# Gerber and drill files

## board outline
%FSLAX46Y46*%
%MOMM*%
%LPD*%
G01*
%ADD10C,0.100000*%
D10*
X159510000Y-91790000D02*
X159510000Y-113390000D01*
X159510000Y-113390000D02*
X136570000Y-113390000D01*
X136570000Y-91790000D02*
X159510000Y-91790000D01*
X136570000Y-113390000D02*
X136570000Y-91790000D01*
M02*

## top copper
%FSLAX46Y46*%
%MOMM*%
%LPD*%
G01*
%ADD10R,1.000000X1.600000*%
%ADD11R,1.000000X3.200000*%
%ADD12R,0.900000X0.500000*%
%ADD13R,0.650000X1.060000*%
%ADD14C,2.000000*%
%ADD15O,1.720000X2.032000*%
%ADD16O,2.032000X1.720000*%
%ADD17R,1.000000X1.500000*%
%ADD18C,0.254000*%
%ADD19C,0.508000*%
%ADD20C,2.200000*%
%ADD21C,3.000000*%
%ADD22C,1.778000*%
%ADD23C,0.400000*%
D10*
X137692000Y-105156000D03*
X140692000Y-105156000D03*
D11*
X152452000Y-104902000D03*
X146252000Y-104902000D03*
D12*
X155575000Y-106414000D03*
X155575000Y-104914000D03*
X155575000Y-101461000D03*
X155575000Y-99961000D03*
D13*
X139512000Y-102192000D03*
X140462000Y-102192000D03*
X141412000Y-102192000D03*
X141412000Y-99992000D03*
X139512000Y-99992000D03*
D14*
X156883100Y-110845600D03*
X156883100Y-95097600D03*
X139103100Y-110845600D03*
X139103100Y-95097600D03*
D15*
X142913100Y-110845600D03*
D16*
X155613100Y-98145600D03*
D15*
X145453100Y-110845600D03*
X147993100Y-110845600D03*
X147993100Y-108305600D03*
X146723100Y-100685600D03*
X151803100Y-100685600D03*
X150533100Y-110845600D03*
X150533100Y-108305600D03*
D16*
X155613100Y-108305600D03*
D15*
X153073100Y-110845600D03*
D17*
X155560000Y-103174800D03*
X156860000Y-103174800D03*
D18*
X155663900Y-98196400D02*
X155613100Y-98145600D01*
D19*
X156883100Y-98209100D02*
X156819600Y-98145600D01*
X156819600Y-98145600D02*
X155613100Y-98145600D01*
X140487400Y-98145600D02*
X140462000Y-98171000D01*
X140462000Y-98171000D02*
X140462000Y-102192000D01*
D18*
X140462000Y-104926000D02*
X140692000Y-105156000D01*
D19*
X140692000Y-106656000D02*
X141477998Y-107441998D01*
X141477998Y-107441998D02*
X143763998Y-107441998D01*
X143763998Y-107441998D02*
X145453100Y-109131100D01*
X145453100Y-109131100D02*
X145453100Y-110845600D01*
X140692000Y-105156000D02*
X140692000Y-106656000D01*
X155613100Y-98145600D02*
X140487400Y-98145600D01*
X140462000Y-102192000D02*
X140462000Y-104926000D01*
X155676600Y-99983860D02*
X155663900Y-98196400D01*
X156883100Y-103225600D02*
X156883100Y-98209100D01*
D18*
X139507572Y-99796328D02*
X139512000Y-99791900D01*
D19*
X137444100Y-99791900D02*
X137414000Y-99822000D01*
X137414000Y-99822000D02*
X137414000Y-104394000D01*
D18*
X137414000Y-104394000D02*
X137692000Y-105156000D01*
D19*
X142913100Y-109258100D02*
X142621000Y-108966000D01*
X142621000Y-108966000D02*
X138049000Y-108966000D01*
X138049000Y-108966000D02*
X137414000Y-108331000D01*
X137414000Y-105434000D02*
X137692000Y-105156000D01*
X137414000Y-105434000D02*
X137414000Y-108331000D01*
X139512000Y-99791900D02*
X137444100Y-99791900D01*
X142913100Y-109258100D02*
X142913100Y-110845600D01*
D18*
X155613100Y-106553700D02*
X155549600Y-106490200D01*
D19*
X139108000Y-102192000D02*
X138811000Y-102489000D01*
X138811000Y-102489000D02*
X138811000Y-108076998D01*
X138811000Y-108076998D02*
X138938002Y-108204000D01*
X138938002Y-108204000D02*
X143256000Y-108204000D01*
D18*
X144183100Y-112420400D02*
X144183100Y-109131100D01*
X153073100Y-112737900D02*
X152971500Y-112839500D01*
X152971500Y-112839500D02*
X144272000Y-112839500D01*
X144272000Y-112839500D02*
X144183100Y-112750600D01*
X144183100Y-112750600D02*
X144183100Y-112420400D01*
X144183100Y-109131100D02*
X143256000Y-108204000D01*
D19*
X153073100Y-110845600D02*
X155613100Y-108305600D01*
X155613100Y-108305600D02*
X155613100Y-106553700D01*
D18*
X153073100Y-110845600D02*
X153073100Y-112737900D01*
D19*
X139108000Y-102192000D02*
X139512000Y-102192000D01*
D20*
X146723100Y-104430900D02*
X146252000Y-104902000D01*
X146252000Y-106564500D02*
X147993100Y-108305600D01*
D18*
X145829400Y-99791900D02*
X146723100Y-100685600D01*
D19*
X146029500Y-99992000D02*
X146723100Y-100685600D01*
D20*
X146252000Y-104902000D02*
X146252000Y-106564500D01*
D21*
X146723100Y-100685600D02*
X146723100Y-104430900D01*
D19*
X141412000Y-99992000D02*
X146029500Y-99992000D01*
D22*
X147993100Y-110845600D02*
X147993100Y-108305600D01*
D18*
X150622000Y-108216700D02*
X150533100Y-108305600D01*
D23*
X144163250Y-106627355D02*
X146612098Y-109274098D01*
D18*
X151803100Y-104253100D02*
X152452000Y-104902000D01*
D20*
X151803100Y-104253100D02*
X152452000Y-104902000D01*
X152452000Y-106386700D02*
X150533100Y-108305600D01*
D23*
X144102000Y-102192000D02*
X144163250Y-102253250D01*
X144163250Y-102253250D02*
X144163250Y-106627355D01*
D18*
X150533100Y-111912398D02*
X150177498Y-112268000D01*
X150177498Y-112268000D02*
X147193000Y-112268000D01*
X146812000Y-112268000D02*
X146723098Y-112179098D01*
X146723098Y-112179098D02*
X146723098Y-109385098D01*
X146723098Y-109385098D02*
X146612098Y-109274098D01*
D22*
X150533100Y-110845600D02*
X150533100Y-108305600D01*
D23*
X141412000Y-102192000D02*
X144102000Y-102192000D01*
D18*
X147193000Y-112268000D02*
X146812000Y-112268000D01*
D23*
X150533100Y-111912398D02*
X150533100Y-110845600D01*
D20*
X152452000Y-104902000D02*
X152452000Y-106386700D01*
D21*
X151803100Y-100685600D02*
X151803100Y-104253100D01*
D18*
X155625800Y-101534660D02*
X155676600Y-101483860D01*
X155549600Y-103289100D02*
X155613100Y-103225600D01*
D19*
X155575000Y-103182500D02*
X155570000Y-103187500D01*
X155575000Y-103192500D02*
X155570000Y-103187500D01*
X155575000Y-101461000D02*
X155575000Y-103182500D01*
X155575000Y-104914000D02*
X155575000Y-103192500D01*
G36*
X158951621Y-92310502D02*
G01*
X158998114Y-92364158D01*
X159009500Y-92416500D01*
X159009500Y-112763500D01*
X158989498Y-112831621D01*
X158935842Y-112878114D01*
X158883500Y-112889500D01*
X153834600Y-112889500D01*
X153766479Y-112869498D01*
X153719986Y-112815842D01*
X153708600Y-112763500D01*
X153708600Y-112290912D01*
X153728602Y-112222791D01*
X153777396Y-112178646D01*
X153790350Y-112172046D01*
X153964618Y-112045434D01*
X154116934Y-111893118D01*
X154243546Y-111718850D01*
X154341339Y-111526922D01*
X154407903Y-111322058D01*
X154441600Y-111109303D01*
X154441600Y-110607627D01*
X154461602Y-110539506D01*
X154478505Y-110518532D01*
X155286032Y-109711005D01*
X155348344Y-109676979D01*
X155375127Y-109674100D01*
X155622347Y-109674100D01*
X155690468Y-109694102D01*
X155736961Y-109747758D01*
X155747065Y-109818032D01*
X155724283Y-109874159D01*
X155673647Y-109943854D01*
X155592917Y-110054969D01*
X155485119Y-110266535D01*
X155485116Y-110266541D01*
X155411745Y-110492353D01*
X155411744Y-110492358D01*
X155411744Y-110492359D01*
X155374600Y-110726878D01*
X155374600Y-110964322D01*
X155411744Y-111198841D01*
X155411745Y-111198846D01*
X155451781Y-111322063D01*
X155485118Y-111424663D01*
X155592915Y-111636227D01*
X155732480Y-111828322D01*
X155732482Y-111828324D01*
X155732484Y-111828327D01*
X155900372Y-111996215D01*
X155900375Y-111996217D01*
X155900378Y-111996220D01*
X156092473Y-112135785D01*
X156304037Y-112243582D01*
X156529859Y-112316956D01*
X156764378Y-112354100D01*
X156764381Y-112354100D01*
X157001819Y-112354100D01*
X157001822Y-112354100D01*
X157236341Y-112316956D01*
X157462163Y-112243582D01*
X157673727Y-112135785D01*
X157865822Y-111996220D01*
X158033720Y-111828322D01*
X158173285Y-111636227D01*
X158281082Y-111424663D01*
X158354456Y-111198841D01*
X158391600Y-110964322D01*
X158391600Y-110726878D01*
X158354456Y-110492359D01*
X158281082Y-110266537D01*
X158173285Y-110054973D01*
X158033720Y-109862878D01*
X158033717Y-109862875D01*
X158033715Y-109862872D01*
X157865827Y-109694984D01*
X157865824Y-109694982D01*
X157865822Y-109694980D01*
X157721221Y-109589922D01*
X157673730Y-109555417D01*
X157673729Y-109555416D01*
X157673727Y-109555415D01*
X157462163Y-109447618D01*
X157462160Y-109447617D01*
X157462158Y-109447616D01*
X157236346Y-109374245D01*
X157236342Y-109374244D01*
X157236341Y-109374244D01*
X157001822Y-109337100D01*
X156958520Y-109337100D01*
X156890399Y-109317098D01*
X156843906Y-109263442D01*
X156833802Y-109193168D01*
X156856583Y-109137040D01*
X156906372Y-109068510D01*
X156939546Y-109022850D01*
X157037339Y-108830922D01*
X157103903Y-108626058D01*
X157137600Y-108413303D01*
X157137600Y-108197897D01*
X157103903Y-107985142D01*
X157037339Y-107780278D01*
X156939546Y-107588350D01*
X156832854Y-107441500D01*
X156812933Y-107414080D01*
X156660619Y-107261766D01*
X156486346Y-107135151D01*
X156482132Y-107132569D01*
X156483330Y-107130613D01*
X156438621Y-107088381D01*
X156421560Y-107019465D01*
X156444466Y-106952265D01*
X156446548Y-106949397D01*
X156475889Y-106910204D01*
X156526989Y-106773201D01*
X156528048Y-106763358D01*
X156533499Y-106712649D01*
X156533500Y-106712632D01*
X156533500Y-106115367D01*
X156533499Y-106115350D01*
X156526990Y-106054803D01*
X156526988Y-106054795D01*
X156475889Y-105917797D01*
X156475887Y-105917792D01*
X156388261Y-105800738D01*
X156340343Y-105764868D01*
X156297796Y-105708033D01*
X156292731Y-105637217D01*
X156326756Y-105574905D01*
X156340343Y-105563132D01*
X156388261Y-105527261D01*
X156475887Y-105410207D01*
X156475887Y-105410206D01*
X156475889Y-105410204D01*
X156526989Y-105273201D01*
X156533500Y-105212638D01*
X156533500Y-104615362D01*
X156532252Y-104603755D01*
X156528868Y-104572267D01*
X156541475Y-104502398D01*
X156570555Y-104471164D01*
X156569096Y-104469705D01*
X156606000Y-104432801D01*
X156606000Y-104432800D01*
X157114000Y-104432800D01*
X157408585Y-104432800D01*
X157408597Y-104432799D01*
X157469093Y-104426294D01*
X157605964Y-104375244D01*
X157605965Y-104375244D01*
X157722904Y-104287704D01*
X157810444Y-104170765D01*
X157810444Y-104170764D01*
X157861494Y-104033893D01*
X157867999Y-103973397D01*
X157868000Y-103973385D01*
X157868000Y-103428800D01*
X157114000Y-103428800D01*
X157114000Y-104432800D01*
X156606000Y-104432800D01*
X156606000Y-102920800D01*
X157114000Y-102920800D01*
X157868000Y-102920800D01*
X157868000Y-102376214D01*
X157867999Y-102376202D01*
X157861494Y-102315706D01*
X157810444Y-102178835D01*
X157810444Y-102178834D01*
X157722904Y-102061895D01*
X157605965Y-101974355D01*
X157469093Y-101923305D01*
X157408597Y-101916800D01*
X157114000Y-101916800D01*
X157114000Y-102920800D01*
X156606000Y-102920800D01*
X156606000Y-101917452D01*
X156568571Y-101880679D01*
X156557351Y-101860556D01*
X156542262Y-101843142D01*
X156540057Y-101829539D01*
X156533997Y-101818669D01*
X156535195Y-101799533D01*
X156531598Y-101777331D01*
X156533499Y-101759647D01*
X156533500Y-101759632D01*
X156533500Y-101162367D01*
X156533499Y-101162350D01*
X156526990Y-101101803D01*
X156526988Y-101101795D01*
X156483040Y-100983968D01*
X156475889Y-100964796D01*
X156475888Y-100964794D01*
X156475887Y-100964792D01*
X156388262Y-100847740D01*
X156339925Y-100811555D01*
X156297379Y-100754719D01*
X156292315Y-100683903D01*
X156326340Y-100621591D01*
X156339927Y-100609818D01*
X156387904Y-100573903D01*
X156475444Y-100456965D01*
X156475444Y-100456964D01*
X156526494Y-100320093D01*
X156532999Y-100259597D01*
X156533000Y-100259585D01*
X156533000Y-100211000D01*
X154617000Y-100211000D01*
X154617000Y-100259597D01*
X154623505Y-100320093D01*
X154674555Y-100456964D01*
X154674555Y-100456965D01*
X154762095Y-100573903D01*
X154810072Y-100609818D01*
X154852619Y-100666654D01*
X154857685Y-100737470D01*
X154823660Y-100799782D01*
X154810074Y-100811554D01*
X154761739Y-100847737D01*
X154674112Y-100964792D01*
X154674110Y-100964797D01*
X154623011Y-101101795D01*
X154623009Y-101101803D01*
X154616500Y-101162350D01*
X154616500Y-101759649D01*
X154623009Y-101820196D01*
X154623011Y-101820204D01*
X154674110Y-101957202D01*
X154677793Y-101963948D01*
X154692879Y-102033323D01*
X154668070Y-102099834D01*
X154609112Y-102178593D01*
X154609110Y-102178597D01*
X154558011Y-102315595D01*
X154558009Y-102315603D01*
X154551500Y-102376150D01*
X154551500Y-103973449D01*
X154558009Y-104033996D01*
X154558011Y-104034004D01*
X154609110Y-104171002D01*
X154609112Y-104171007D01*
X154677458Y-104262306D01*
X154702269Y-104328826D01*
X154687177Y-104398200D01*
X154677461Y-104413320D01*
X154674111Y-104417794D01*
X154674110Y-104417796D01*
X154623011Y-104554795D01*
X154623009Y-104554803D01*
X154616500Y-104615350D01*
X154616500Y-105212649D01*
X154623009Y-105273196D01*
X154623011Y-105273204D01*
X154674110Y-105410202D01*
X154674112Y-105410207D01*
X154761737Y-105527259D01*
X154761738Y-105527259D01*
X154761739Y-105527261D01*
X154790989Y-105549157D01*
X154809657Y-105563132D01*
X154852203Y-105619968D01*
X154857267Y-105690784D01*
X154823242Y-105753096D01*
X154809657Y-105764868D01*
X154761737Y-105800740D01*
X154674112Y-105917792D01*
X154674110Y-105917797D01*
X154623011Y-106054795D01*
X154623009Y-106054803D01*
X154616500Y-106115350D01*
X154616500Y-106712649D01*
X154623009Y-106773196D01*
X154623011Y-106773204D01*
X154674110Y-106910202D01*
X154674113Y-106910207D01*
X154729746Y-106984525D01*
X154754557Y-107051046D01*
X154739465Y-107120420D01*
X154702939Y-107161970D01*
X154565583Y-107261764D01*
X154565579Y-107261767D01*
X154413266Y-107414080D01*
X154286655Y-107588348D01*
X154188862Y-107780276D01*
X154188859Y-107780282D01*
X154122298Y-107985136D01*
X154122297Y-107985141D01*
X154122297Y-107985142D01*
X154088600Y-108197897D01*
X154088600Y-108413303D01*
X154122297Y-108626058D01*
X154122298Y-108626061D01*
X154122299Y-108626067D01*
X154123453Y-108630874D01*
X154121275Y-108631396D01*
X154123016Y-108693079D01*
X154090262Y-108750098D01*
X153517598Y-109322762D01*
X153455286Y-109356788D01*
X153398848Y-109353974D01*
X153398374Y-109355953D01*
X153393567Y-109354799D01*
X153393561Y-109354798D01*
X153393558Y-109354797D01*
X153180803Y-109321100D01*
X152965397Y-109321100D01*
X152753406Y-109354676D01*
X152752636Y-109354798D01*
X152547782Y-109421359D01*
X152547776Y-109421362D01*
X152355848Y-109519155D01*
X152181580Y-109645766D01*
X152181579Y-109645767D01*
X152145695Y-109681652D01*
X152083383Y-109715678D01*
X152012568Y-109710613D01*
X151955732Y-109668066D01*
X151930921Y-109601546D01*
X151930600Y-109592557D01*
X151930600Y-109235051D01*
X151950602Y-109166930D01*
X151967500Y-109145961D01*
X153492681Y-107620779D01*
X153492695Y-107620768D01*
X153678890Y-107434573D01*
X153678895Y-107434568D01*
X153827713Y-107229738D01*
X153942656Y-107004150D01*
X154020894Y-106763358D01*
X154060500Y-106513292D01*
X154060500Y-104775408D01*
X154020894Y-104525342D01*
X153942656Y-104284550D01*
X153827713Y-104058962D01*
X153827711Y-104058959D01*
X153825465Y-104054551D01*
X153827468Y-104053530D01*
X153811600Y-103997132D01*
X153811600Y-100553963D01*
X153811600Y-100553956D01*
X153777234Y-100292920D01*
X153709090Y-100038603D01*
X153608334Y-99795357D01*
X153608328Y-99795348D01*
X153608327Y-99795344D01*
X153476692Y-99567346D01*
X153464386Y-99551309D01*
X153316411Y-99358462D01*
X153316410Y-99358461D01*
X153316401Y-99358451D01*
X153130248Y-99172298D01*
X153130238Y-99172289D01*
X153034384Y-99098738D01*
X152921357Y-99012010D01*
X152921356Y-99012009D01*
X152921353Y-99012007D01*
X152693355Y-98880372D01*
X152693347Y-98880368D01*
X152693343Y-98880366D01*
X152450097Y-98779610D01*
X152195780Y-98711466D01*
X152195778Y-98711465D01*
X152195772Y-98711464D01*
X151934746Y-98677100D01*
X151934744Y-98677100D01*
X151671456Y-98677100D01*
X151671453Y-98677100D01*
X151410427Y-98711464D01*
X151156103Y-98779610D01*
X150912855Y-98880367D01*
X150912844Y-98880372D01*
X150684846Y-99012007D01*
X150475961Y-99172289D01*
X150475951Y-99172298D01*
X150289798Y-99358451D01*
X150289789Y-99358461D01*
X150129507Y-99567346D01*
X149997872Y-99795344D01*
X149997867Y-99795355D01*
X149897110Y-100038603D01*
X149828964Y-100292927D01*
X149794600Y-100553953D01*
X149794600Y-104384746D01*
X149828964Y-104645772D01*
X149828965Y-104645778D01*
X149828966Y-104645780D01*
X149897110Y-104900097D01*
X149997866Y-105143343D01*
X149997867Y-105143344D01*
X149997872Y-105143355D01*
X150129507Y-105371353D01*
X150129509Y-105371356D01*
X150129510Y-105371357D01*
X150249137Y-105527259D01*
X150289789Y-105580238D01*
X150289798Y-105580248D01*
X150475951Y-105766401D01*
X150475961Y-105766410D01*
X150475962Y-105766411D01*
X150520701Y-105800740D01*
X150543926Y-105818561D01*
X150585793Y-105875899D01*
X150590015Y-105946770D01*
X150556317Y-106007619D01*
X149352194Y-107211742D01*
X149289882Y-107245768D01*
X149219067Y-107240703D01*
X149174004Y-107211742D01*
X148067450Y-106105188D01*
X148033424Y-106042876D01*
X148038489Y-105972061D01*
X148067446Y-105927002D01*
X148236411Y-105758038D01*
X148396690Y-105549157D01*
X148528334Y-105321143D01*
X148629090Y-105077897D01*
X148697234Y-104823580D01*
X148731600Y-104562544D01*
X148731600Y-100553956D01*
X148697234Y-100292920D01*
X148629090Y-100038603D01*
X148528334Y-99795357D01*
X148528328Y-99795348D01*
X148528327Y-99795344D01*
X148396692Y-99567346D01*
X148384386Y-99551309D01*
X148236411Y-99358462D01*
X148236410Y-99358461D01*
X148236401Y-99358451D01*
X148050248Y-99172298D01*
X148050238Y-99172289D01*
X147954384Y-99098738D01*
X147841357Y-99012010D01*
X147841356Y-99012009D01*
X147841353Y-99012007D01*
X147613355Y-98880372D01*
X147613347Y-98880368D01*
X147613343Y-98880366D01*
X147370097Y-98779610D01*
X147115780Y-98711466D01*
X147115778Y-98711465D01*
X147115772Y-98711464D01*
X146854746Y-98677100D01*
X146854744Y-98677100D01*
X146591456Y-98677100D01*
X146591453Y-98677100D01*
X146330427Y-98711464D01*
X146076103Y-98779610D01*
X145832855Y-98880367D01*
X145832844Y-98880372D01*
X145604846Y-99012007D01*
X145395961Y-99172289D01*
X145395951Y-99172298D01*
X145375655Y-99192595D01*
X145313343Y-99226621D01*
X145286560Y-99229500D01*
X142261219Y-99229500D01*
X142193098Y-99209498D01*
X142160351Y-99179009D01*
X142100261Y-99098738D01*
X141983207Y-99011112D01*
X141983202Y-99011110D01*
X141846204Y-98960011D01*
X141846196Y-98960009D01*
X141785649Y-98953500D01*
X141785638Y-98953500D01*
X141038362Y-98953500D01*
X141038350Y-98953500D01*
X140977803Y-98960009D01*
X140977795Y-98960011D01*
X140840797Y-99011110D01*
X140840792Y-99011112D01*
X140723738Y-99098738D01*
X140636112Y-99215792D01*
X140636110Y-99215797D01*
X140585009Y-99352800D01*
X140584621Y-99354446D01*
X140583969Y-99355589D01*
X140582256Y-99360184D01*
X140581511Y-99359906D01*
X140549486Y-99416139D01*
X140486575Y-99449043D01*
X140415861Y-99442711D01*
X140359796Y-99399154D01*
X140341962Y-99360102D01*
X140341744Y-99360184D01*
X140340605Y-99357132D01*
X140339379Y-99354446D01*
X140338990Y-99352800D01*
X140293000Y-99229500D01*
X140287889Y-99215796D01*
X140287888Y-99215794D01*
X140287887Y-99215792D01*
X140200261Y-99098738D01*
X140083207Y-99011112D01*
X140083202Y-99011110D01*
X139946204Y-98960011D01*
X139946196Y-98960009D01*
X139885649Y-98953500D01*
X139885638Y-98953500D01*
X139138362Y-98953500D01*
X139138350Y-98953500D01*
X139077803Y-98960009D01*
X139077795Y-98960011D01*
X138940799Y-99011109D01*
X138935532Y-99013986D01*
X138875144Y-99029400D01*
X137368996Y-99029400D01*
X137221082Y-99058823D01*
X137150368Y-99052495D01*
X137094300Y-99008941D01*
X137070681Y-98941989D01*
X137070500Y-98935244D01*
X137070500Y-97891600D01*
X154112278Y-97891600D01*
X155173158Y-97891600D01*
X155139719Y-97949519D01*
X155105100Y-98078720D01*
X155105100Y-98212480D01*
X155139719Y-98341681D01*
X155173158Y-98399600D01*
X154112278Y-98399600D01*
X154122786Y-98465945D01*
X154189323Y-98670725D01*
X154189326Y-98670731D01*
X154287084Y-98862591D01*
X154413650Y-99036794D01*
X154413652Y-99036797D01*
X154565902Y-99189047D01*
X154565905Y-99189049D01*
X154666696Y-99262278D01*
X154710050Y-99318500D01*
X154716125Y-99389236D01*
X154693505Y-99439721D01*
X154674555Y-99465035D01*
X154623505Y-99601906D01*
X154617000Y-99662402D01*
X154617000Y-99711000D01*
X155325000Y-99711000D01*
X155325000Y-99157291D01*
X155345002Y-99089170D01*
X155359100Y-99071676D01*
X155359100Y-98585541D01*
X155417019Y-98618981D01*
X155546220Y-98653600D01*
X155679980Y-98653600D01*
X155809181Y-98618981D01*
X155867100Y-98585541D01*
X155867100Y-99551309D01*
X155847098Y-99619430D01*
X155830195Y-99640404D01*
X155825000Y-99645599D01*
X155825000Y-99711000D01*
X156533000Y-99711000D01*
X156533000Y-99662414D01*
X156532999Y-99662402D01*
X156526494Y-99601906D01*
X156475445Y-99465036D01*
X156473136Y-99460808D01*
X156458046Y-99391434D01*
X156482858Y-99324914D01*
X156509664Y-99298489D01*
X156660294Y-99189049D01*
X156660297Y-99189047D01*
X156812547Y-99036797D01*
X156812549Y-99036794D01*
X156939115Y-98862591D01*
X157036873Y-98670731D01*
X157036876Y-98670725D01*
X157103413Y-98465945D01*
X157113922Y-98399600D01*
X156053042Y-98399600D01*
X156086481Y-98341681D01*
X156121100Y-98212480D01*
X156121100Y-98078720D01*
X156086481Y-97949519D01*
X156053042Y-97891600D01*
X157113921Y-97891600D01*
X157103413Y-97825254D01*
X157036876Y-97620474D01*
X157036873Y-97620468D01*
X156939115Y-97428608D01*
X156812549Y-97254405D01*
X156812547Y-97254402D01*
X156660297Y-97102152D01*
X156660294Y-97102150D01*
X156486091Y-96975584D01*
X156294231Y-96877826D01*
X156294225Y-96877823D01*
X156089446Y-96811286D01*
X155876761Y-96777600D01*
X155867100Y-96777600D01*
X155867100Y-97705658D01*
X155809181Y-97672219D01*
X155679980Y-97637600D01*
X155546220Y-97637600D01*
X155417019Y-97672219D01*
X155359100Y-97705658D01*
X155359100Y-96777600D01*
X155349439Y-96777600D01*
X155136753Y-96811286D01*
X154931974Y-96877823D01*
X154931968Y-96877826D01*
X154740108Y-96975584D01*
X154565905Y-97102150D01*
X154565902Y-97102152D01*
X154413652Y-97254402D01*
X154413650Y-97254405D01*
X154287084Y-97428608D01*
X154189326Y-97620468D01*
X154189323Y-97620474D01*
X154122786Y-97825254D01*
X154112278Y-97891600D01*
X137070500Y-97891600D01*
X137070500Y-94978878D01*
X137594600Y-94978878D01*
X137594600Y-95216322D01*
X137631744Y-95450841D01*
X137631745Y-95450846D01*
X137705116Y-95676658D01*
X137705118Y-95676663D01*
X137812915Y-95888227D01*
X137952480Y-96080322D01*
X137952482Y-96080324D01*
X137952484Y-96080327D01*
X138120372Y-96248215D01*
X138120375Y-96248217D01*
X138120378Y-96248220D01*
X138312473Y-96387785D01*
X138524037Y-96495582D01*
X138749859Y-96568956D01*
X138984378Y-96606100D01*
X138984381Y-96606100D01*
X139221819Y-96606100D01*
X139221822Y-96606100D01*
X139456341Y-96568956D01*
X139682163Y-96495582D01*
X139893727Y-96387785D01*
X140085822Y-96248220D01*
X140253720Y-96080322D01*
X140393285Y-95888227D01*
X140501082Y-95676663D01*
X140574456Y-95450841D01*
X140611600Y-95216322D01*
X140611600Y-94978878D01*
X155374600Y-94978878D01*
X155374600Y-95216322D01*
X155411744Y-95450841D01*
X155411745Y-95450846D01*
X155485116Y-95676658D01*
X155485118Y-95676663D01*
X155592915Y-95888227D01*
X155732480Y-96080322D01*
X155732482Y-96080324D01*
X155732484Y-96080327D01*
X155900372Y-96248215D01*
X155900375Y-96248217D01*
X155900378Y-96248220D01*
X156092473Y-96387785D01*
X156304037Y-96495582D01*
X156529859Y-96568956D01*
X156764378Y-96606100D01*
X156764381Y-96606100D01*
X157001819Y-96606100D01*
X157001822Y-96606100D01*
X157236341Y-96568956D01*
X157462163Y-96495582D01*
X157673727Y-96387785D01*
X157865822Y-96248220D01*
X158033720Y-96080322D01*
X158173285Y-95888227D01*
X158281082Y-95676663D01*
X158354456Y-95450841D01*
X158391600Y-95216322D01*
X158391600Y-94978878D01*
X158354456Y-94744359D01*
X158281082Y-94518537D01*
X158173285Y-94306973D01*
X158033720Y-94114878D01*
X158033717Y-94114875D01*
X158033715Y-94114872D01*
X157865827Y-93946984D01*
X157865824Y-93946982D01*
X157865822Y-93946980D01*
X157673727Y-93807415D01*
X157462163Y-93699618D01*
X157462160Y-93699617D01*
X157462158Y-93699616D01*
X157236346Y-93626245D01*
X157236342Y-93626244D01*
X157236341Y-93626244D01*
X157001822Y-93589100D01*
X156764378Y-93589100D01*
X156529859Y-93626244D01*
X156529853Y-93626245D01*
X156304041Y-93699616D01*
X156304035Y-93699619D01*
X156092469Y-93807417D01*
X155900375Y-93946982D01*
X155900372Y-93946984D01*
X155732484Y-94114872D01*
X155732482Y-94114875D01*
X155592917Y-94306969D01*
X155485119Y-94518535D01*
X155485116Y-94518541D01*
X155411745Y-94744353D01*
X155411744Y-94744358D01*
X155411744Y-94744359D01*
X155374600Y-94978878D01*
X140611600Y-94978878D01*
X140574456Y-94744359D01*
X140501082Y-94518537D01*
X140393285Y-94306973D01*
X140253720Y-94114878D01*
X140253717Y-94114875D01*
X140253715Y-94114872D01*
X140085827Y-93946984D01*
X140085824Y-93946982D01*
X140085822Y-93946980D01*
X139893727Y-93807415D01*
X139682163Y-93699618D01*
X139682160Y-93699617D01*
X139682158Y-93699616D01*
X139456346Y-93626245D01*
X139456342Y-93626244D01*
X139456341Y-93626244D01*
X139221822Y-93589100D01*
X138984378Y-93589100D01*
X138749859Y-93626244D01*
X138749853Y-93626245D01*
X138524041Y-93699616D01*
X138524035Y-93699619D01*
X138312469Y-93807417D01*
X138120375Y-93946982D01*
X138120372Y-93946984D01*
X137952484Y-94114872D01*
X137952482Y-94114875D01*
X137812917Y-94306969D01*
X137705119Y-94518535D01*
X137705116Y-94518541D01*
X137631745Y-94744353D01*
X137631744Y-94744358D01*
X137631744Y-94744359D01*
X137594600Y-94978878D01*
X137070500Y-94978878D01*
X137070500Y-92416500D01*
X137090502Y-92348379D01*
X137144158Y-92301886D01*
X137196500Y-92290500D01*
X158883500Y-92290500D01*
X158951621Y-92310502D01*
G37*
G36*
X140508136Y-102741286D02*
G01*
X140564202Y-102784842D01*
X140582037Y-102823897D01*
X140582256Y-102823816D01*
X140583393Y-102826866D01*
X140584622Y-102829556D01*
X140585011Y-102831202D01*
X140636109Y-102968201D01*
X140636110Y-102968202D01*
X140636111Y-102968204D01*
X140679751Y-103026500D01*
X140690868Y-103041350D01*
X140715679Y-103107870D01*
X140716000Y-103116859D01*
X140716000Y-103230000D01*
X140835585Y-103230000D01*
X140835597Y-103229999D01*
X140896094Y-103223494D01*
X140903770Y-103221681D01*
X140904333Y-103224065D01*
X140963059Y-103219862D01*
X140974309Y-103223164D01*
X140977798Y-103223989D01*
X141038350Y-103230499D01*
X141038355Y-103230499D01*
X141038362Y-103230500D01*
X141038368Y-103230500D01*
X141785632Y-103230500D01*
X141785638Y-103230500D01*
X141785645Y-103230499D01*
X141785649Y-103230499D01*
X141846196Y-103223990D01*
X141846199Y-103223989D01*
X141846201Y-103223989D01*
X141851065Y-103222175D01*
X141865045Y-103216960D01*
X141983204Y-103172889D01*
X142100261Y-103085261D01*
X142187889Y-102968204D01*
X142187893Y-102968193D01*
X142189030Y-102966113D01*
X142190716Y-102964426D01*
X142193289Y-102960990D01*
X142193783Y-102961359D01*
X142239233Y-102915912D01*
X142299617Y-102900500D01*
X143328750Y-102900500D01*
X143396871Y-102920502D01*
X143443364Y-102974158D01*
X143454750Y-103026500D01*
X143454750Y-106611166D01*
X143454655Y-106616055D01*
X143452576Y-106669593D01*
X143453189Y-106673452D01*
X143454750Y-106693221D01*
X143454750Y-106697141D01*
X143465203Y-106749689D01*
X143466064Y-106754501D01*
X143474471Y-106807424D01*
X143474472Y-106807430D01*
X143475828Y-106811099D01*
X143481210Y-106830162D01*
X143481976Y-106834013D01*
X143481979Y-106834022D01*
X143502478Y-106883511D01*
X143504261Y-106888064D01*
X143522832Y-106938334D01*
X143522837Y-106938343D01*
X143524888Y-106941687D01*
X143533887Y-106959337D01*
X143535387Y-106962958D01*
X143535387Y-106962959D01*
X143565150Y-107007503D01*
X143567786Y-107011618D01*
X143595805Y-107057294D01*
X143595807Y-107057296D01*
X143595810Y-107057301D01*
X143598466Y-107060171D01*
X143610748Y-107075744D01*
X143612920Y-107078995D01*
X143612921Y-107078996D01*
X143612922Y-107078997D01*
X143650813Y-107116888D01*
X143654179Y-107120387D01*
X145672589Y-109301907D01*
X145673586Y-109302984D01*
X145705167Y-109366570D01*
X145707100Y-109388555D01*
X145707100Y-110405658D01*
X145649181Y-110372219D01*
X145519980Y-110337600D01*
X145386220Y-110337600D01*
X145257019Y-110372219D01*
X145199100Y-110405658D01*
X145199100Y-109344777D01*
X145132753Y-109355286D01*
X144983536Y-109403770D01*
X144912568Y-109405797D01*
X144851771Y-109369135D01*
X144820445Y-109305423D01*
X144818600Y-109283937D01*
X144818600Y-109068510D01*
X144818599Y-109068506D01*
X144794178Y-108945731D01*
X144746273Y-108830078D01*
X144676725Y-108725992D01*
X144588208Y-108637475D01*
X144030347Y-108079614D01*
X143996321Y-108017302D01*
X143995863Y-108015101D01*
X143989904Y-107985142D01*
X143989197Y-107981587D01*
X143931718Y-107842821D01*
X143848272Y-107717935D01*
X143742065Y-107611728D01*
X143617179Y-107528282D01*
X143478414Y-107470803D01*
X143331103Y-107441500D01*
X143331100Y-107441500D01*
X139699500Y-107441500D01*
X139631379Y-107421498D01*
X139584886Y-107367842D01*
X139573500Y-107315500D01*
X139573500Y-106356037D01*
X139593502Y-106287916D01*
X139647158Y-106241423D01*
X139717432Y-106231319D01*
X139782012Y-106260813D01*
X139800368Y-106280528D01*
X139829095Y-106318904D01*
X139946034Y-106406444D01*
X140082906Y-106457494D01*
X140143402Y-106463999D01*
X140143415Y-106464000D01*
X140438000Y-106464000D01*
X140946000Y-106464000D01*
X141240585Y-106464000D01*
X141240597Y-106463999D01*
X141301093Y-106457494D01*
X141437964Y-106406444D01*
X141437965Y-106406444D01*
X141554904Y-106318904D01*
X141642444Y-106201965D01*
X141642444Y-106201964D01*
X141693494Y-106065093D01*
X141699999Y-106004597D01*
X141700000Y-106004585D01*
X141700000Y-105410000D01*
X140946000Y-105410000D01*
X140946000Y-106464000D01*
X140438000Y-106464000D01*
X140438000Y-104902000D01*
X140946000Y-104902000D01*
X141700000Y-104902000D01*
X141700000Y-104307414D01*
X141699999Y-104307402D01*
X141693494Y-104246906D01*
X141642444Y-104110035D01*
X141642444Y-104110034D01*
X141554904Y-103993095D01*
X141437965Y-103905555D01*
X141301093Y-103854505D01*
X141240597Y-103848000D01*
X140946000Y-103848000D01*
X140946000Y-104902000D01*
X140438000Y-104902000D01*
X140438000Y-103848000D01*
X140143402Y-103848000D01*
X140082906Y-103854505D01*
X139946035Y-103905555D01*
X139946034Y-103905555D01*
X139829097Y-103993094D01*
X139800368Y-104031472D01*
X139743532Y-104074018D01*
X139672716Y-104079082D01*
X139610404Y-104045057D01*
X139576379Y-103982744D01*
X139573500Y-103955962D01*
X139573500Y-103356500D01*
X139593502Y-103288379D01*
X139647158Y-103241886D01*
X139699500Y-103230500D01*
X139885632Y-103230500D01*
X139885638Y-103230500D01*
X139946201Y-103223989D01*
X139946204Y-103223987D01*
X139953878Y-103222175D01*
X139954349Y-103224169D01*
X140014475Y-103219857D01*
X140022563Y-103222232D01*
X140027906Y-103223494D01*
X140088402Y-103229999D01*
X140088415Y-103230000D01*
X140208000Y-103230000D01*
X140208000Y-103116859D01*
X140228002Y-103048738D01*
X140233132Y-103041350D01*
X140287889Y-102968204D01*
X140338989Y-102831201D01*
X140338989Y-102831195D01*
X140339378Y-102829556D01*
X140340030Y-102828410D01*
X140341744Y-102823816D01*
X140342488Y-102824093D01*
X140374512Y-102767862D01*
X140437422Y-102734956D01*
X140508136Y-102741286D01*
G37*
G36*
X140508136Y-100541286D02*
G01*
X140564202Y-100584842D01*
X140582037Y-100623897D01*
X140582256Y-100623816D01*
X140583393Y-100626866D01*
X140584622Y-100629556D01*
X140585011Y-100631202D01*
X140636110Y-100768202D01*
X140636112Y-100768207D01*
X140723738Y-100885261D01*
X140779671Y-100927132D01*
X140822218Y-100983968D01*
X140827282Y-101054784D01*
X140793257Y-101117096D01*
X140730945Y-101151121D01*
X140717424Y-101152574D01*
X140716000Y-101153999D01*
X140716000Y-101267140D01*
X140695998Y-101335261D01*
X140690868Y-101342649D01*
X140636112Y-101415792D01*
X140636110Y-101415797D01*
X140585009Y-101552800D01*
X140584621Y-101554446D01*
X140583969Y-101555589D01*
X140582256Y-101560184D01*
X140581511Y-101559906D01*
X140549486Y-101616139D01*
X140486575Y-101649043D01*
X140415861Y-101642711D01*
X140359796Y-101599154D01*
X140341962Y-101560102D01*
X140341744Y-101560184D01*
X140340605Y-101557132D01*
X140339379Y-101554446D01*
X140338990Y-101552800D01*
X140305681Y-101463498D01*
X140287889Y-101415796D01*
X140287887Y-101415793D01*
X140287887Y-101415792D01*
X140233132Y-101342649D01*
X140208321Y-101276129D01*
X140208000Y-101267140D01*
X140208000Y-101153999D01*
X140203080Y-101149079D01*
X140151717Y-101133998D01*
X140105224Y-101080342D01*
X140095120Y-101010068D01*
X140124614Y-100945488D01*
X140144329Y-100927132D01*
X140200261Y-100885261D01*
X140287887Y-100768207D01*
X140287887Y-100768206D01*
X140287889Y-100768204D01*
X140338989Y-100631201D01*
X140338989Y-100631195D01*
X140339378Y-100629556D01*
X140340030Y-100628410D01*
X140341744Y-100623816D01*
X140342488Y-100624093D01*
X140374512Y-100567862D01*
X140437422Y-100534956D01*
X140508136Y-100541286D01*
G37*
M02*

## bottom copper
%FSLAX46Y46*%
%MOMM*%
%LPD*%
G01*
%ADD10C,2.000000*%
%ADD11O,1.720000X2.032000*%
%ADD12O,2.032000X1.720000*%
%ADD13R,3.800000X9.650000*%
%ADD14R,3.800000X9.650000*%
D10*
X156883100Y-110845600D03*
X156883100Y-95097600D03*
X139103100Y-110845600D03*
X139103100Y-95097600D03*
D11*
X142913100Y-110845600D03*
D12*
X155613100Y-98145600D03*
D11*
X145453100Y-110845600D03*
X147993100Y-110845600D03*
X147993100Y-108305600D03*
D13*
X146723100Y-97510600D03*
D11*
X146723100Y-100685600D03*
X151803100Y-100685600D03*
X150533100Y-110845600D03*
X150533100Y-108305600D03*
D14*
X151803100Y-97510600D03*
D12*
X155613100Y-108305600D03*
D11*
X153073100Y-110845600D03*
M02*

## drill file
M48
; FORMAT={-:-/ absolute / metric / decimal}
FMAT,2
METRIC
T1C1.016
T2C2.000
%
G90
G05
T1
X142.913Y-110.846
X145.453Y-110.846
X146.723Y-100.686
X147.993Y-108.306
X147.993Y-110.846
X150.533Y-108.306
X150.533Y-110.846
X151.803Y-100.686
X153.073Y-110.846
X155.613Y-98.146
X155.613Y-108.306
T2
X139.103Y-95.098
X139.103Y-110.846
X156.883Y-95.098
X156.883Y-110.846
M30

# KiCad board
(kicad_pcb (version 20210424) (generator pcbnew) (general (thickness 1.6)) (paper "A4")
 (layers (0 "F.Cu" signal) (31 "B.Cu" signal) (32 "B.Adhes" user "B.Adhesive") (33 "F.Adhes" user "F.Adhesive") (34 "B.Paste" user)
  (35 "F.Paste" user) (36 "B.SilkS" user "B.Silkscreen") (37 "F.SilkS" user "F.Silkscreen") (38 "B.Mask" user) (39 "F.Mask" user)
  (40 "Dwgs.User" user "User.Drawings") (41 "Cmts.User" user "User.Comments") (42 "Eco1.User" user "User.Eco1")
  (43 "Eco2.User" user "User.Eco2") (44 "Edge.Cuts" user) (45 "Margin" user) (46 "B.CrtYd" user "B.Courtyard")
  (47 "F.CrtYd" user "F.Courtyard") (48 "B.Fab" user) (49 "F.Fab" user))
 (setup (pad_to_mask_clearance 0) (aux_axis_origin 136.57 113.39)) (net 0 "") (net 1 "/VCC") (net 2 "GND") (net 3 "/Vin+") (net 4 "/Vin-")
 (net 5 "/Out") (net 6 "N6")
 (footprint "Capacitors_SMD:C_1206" (layer "F.Cu") (at 139.192 105.156)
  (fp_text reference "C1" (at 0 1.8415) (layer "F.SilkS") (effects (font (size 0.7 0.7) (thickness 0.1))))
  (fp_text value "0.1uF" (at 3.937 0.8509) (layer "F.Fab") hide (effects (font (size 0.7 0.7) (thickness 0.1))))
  (pad "1" smd rect locked (at -1.5 0) (size 1 1.6) (layers "F.Cu" "F.Paste" "F.Mask") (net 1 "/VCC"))
  (pad "2" smd rect locked (at 1.5 0) (size 1 1.6) (layers "F.Cu" "F.Paste" "F.Mask") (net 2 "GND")))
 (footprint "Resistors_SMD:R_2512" (layer "F.Cu") (at 149.352 104.902 180)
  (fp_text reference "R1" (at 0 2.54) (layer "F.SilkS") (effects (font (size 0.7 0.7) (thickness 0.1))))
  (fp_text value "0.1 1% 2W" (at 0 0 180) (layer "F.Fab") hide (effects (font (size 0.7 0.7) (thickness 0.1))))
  (pad "1" smd rect locked (at -3.1 0 180) (size 1 3.2) (layers "F.Cu" "F.Paste" "F.Mask") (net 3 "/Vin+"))
  (pad "2" smd rect locked (at 3.1 0 180) (size 1 3.2) (layers "F.Cu" "F.Paste" "F.Mask") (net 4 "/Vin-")))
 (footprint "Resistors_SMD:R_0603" (layer "F.Cu") (at 155.575 105.664 90)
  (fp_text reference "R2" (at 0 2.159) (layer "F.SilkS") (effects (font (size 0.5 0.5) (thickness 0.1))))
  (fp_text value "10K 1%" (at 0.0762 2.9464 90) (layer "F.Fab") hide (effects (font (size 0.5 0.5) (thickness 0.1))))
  (pad "1" smd rect locked (at -0.75 0 90) (size 0.5 0.9) (layers "F.Cu" "F.Paste" "F.Mask") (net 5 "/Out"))
  (pad "2" smd rect locked (at 0.75 0 90) (size 0.5 0.9) (layers "F.Cu" "F.Paste" "F.Mask") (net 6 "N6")))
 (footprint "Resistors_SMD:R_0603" (layer "F.Cu") (at 155.575 100.711 90)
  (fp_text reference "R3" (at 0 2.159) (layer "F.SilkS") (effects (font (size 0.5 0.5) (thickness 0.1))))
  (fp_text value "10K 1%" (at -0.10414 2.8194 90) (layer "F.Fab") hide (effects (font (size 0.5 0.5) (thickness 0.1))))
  (pad "1" smd rect locked (at -0.75 0 90) (size 0.5 0.9) (layers "F.Cu" "F.Paste" "F.Mask") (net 6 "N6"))
  (pad "2" smd rect locked (at 0.75 0 90) (size 0.5 0.9) (layers "F.Cu" "F.Paste" "F.Mask") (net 2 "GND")))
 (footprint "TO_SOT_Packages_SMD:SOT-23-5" (layer "F.Cu") (at 140.462 101.092 90)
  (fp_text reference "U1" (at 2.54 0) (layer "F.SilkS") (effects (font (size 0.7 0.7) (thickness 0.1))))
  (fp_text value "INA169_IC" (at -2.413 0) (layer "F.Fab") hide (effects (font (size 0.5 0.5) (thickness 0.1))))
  (pad "1" smd rect locked (at -1.1 -0.95 90) (size 1.06 0.65) (layers "F.Cu" "F.Paste" "F.Mask") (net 5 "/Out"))
  (pad "2" smd rect locked (at -1.1 0 90) (size 1.06 0.65) (layers "F.Cu" "F.Paste" "F.Mask") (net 2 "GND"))
  (pad "3" smd rect locked (at -1.1 0.95 90) (size 1.06 0.65) (layers "F.Cu" "F.Paste" "F.Mask") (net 3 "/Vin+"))
  (pad "4" smd rect locked (at 1.1 0.95 90) (size 1.06 0.65) (layers "F.Cu" "F.Paste" "F.Mask") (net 4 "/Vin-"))
  (pad "5" smd rect locked (at 1.1 -0.95 90) (size 1.06 0.65) (layers "F.Cu" "F.Paste" "F.Mask") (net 1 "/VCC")))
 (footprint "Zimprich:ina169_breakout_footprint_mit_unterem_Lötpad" (layer "F.Cu") (at 147.9931 103.2256)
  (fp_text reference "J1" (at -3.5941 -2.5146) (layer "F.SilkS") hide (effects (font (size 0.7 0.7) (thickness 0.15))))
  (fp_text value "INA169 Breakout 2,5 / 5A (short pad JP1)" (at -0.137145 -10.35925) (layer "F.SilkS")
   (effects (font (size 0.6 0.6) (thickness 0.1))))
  (pad "" thru_hole circle locked (at 8.89 7.62) (size 2 2) (drill 2) (layers *.Cu *.Mask "F.SilkS"))
  (pad "" thru_hole circle locked (at 8.89 -8.128) (size 2 2) (drill 2) (layers *.Cu *.Mask "F.SilkS"))
  (pad "" thru_hole circle locked (at -8.89 7.62) (size 2 2) (drill 2) (layers *.Cu *.Mask "F.SilkS"))
  (pad "" thru_hole circle locked (at -8.89 -8.128) (size 2 2) (drill 2) (layers *.Cu *.Mask "F.SilkS"))
  (pad "1" thru_hole oval locked (at -5.08 7.62) (size 1.72 2.032) (drill 1.016) (layers *.Cu *.Mask "F.SilkS") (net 1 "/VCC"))
  (pad "2" thru_hole oval locked (at 7.62 -5.08) (size 2.032 1.72) (drill 1.016) (layers *.Cu *.Mask "F.SilkS") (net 2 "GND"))
  (pad "2" thru_hole oval locked (at -2.54 7.62) (size 1.72 2.032) (drill 1.016) (layers *.Cu *.Mask "F.SilkS") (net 2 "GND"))
  (pad "3" thru_hole oval locked (at 0 7.62) (size 1.72 2.032) (drill 1.016) (layers *.Cu *.Mask "F.SilkS") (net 4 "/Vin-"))
  (pad "3" thru_hole oval locked (at 0 5.08) (size 1.72 2.032) (drill 1.016) (layers *.Cu *.Mask "F.SilkS") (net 4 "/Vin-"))
  (pad "3" connect rect locked (at -1.27 -5.715) (size 3.8 9.65) (layers "B.Cu" "B.Mask") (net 4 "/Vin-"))
  (pad "3" thru_hole oval locked (at -1.27 -2.54) (size 1.72 2.032) (drill 1.016) (layers *.Cu *.Mask "F.SilkS") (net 4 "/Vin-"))
  (pad "4" thru_hole oval locked (at 3.81 -2.54) (size 1.72 2.032) (drill 1.016) (layers *.Cu *.Mask "F.SilkS") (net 3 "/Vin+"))
  (pad "4" thru_hole oval locked (at 2.54 7.62) (size 1.72 2.032) (drill 1.016) (layers *.Cu *.Mask "F.SilkS") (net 3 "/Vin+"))
  (pad "4" thru_hole oval locked (at 2.54 5.08) (size 1.72 2.032) (drill 1.016) (layers *.Cu *.Mask "F.SilkS") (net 3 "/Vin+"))
  (pad "4" smd rect locked (at 3.81 -5.715) (size 3.8 9.65) (layers "B.Cu" "B.Mask") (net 3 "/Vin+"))
  (pad "5" thru_hole oval locked (at 7.62 5.08) (size 2.032 1.72) (drill 1.016) (layers *.Cu *.Mask "F.SilkS") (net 5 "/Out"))
  (pad "5" thru_hole oval locked (at 5.08 7.62) (size 1.72 2.032) (drill 1.016) (layers *.Cu *.Mask "F.SilkS") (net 5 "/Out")))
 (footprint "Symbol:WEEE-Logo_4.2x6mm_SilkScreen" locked (layer "F.Cu") (at 143.129 106.172)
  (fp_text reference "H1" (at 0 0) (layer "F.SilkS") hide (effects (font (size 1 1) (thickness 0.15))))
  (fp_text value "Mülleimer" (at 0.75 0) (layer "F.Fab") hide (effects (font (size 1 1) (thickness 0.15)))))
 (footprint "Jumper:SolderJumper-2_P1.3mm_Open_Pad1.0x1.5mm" (layer "F.Cu") (at 156.21 103.1748)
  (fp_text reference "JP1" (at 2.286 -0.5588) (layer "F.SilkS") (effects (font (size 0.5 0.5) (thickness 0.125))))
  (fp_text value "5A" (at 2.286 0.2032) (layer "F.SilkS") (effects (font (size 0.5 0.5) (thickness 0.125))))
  (pad "1" smd rect locked (at -0.65 0) (size 1 1.5) (layers "F.Cu" "F.Mask") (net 6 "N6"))
  (pad "2" smd rect locked (at 0.65 0) (size 1 1.5) (layers "F.Cu" "F.Mask") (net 2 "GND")))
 (gr_line (start 159.51 91.79) (end 159.51 113.39) (angle 90) (layer "Edge.Cuts") (width 0.1))
 (gr_line (start 159.51 113.39) (end 136.57 113.39) (angle 90) (layer "Edge.Cuts") (width 0.1))
 (gr_line (start 136.57 91.79) (end 159.51 91.79) (angle 90) (layer "Edge.Cuts") (width 0.1))
 (gr_line (start 136.57 113.39) (end 136.57 91.79) (angle 90) (layer "Edge.Cuts") (width 0.1))
 (segment (start 155.6639 98.1964) (end 155.6131 98.1456) (width 0.254) (layer "F.Cu") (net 2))
 (segment (start 156.8831 98.2091) (end 156.8196 98.1456) (width 0.508) (layer "F.Cu") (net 2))
 (segment (start 156.8196 98.1456) (end 155.6131 98.1456) (width 0.508) (layer "F.Cu") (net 2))
 (segment (start 140.4874 98.1456) (end 140.462 98.171) (width 0.508) (layer "F.Cu") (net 2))
 (segment (start 140.462 98.171) (end 140.462 102.192) (width 0.508) (layer "F.Cu") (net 2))
 (segment (start 140.462 104.926) (end 140.692 105.156) (width 0.254) (layer "F.Cu") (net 2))
 (segment (start 140.692 106.656) (end 141.477998 107.441998) (width 0.508) (layer "F.Cu") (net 2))
 (segment (start 141.477998 107.441998) (end 143.763998 107.441998) (width 0.508) (layer "F.Cu") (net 2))
 (segment (start 143.763998 107.441998) (end 145.4531 109.1311) (width 0.508) (layer "F.Cu") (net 2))
 (segment (start 145.4531 109.1311) (end 145.4531 110.8456) (width 0.508) (layer "F.Cu") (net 2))
 (segment (start 140.692 105.156) (end 140.692 106.656) (width 0.508) (layer "F.Cu") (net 2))
 (segment (start 155.6131 98.1456) (end 140.4874 98.1456) (width 0.508) (layer "F.Cu") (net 2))
 (segment (start 140.462 102.192) (end 140.462 104.926) (width 0.508) (layer "F.Cu") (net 2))
 (segment (start 155.6766 99.98386) (end 155.6639 98.1964) (width 0.508) (layer "F.Cu") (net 2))
 (segment (start 156.8831 103.2256) (end 156.8831 98.2091) (width 0.508) (layer "F.Cu") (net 2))
 (segment (start 139.507572 99.796328) (end 139.512 99.7919) (width 0.254) (layer "F.Cu") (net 1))
 (segment (start 137.4441 99.7919) (end 137.414 99.822) (width 0.508) (layer "F.Cu") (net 1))
 (segment (start 137.414 99.822) (end 137.414 104.394) (width 0.508) (layer "F.Cu") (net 1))
 (segment (start 137.414 104.394) (end 137.692 105.156) (width 0.254) (layer "F.Cu") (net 1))
 (segment (start 142.9131 109.2581) (end 142.621 108.966) (width 0.508) (layer "F.Cu") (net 1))
 (segment (start 142.621 108.966) (end 138.049 108.966) (width 0.508) (layer "F.Cu") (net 1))
 (segment (start 138.049 108.966) (end 137.414 108.331) (width 0.508) (layer "F.Cu") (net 1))
 (segment (start 137.414 105.434) (end 137.692 105.156) (width 0.508) (layer "F.Cu") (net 1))
 (segment (start 137.414 105.434) (end 137.414 108.331) (width 0.508) (layer "F.Cu") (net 1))
 (segment (start 139.512 99.7919) (end 137.4441 99.7919) (width 0.508) (layer "F.Cu") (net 1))
 (segment (start 142.9131 109.2581) (end 142.9131 110.8456) (width 0.508) (layer "F.Cu") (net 1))
 (segment (start 155.6131 106.5537) (end 155.5496 106.4902) (width 0.254) (layer "F.Cu") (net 5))
 (segment (start 139.108 102.192) (end 138.811 102.489) (width 0.508) (layer "F.Cu") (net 5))
 (segment (start 138.811 102.489) (end 138.811 108.076998) (width 0.508) (layer "F.Cu") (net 5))
 (segment (start 138.811 108.076998) (end 138.938002 108.204) (width 0.508) (layer "F.Cu") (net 5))
 (segment (start 138.938002 108.204) (end 143.256 108.204) (width 0.508) (layer "F.Cu") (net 5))
 (segment (start 144.1831 112.4204) (end 144.1831 109.1311) (width 0.254) (layer "F.Cu") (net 5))
 (segment (start 153.0731 112.7379) (end 152.9715 112.8395) (width 0.254) (layer "F.Cu") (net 5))
 (segment (start 152.9715 112.8395) (end 144.272 112.8395) (width 0.254) (layer "F.Cu") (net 5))
 (segment (start 144.272 112.8395) (end 144.1831 112.7506) (width 0.254) (layer "F.Cu") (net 5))
 (segment (start 144.1831 112.7506) (end 144.1831 112.4204) (width 0.254) (layer "F.Cu") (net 5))
 (segment (start 144.1831 109.1311) (end 143.256 108.204) (width 0.254) (layer "F.Cu") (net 5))
 (segment (start 153.0731 110.8456) (end 155.6131 108.3056) (width 0.508) (layer "F.Cu") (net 5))
 (segment (start 155.6131 108.3056) (end 155.6131 106.5537) (width 0.508) (layer "F.Cu") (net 5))
 (segment (start 153.0731 110.8456) (end 153.0731 112.7379) (width 0.254) (layer "F.Cu") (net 5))
 (segment (start 139.108 102.192) (end 139.512 102.192) (width 0.508) (layer "F.Cu") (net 5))
 (segment (start 146.7231 104.4309) (end 146.252 104.902) (width 2.2) (layer "F.Cu") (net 4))
 (segment (start 146.252 106.5645) (end 147.9931 108.3056) (width 2.2) (layer "F.Cu") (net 4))
 (segment (start 145.8294 99.7919) (end 146.7231 100.6856) (width 0.254) (layer "F.Cu") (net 4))
 (segment (start 146.0295 99.992) (end 146.7231 100.6856) (width 0.508) (layer "F.Cu") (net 4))
 (segment (start 146.252 104.902) (end 146.252 106.5645) (width 2.2) (layer "F.Cu") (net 4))
 (segment (start 146.7231 100.6856) (end 146.7231 104.4309) (width 3) (layer "F.Cu") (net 4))
 (segment (start 141.412 99.992) (end 146.0295 99.992) (width 0.508) (layer "F.Cu") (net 4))
 (segment (start 147.9931 110.8456) (end 147.9931 108.3056) (width 1.778) (layer "F.Cu") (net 4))
 (segment (start 150.622 108.2167) (end 150.5331 108.3056) (width 0.254) (layer "F.Cu") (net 3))
 (segment (start 144.16325 106.627355) (end 146.612098 109.274098) (width 0.4) (layer "F.Cu") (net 3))
 (segment (start 151.8031 104.2531) (end 152.452 104.902) (width 0.254) (layer "F.Cu") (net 3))
 (segment (start 151.8031 104.2531) (end 152.452 104.902) (width 2.2) (layer "F.Cu") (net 3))
 (segment (start 152.452 106.3867) (end 150.5331 108.3056) (width 2.2) (layer "F.Cu") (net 3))
 (segment (start 144.102 102.192) (end 144.16325 102.25325) (width 0.4) (layer "F.Cu") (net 3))
 (segment (start 144.16325 102.25325) (end 144.16325 106.627355) (width 0.4) (layer "F.Cu") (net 3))
 (segment (start 150.5331 111.912398) (end 150.177498 112.268) (width 0.254) (layer "F.Cu") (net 3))
 (segment (start 150.177498 112.268) (end 147.193 112.268) (width 0.254) (layer "F.Cu") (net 3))
 (segment (start 146.812 112.268) (end 146.723098 112.179098) (width 0.254) (layer "F.Cu") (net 3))
 (segment (start 146.723098 112.179098) (end 146.723098 109.385098) (width 0.254) (layer "F.Cu") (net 3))
 (segment (start 146.723098 109.385098) (end 146.612098 109.274098) (width 0.254) (layer "F.Cu") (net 3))
 (segment (start 150.5331 110.8456) (end 150.5331 108.3056) (width 1.778) (layer "F.Cu") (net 3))
 (segment (start 141.412 102.192) (end 144.102 102.192) (width 0.4) (layer "F.Cu") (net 3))
 (segment (start 147.193 112.268) (end 146.812 112.268) (width 0.254) (layer "F.Cu") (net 3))
 (segment (start 150.5331 111.912398) (end 150.5331 110.8456) (width 0.4) (layer "F.Cu") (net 3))
 (segment (start 152.452 104.902) (end 152.452 106.3867) (width 2.2) (layer "F.Cu") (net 3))
 (segment (start 151.8031 100.6856) (end 151.8031 104.2531) (width 3) (layer "F.Cu") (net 3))
 (segment (start 155.6258 101.53466) (end 155.6766 101.48386) (width 0.254) (layer "F.Cu") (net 6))
 (segment (start 155.5496 103.2891) (end 155.6131 103.2256) (width 0.254) (layer "F.Cu") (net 6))
 (segment (start 155.575 103.1825) (end 155.57 103.1875) (width 0.508) (layer "F.Cu") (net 6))
 (segment (start 155.575 103.1925) (end 155.57 103.1875) (width 0.508) (layer "F.Cu") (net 6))
 (segment (start 155.575 101.461) (end 155.575 103.1825) (width 0.508) (layer "F.Cu") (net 6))
 (segment (start 155.575 104.914) (end 155.575 103.1925) (width 0.508) (layer "F.Cu") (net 6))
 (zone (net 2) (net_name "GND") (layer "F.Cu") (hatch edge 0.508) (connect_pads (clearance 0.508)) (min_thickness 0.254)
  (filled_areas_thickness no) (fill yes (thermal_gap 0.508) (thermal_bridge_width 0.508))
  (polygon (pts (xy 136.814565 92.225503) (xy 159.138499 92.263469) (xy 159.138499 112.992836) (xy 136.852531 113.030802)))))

